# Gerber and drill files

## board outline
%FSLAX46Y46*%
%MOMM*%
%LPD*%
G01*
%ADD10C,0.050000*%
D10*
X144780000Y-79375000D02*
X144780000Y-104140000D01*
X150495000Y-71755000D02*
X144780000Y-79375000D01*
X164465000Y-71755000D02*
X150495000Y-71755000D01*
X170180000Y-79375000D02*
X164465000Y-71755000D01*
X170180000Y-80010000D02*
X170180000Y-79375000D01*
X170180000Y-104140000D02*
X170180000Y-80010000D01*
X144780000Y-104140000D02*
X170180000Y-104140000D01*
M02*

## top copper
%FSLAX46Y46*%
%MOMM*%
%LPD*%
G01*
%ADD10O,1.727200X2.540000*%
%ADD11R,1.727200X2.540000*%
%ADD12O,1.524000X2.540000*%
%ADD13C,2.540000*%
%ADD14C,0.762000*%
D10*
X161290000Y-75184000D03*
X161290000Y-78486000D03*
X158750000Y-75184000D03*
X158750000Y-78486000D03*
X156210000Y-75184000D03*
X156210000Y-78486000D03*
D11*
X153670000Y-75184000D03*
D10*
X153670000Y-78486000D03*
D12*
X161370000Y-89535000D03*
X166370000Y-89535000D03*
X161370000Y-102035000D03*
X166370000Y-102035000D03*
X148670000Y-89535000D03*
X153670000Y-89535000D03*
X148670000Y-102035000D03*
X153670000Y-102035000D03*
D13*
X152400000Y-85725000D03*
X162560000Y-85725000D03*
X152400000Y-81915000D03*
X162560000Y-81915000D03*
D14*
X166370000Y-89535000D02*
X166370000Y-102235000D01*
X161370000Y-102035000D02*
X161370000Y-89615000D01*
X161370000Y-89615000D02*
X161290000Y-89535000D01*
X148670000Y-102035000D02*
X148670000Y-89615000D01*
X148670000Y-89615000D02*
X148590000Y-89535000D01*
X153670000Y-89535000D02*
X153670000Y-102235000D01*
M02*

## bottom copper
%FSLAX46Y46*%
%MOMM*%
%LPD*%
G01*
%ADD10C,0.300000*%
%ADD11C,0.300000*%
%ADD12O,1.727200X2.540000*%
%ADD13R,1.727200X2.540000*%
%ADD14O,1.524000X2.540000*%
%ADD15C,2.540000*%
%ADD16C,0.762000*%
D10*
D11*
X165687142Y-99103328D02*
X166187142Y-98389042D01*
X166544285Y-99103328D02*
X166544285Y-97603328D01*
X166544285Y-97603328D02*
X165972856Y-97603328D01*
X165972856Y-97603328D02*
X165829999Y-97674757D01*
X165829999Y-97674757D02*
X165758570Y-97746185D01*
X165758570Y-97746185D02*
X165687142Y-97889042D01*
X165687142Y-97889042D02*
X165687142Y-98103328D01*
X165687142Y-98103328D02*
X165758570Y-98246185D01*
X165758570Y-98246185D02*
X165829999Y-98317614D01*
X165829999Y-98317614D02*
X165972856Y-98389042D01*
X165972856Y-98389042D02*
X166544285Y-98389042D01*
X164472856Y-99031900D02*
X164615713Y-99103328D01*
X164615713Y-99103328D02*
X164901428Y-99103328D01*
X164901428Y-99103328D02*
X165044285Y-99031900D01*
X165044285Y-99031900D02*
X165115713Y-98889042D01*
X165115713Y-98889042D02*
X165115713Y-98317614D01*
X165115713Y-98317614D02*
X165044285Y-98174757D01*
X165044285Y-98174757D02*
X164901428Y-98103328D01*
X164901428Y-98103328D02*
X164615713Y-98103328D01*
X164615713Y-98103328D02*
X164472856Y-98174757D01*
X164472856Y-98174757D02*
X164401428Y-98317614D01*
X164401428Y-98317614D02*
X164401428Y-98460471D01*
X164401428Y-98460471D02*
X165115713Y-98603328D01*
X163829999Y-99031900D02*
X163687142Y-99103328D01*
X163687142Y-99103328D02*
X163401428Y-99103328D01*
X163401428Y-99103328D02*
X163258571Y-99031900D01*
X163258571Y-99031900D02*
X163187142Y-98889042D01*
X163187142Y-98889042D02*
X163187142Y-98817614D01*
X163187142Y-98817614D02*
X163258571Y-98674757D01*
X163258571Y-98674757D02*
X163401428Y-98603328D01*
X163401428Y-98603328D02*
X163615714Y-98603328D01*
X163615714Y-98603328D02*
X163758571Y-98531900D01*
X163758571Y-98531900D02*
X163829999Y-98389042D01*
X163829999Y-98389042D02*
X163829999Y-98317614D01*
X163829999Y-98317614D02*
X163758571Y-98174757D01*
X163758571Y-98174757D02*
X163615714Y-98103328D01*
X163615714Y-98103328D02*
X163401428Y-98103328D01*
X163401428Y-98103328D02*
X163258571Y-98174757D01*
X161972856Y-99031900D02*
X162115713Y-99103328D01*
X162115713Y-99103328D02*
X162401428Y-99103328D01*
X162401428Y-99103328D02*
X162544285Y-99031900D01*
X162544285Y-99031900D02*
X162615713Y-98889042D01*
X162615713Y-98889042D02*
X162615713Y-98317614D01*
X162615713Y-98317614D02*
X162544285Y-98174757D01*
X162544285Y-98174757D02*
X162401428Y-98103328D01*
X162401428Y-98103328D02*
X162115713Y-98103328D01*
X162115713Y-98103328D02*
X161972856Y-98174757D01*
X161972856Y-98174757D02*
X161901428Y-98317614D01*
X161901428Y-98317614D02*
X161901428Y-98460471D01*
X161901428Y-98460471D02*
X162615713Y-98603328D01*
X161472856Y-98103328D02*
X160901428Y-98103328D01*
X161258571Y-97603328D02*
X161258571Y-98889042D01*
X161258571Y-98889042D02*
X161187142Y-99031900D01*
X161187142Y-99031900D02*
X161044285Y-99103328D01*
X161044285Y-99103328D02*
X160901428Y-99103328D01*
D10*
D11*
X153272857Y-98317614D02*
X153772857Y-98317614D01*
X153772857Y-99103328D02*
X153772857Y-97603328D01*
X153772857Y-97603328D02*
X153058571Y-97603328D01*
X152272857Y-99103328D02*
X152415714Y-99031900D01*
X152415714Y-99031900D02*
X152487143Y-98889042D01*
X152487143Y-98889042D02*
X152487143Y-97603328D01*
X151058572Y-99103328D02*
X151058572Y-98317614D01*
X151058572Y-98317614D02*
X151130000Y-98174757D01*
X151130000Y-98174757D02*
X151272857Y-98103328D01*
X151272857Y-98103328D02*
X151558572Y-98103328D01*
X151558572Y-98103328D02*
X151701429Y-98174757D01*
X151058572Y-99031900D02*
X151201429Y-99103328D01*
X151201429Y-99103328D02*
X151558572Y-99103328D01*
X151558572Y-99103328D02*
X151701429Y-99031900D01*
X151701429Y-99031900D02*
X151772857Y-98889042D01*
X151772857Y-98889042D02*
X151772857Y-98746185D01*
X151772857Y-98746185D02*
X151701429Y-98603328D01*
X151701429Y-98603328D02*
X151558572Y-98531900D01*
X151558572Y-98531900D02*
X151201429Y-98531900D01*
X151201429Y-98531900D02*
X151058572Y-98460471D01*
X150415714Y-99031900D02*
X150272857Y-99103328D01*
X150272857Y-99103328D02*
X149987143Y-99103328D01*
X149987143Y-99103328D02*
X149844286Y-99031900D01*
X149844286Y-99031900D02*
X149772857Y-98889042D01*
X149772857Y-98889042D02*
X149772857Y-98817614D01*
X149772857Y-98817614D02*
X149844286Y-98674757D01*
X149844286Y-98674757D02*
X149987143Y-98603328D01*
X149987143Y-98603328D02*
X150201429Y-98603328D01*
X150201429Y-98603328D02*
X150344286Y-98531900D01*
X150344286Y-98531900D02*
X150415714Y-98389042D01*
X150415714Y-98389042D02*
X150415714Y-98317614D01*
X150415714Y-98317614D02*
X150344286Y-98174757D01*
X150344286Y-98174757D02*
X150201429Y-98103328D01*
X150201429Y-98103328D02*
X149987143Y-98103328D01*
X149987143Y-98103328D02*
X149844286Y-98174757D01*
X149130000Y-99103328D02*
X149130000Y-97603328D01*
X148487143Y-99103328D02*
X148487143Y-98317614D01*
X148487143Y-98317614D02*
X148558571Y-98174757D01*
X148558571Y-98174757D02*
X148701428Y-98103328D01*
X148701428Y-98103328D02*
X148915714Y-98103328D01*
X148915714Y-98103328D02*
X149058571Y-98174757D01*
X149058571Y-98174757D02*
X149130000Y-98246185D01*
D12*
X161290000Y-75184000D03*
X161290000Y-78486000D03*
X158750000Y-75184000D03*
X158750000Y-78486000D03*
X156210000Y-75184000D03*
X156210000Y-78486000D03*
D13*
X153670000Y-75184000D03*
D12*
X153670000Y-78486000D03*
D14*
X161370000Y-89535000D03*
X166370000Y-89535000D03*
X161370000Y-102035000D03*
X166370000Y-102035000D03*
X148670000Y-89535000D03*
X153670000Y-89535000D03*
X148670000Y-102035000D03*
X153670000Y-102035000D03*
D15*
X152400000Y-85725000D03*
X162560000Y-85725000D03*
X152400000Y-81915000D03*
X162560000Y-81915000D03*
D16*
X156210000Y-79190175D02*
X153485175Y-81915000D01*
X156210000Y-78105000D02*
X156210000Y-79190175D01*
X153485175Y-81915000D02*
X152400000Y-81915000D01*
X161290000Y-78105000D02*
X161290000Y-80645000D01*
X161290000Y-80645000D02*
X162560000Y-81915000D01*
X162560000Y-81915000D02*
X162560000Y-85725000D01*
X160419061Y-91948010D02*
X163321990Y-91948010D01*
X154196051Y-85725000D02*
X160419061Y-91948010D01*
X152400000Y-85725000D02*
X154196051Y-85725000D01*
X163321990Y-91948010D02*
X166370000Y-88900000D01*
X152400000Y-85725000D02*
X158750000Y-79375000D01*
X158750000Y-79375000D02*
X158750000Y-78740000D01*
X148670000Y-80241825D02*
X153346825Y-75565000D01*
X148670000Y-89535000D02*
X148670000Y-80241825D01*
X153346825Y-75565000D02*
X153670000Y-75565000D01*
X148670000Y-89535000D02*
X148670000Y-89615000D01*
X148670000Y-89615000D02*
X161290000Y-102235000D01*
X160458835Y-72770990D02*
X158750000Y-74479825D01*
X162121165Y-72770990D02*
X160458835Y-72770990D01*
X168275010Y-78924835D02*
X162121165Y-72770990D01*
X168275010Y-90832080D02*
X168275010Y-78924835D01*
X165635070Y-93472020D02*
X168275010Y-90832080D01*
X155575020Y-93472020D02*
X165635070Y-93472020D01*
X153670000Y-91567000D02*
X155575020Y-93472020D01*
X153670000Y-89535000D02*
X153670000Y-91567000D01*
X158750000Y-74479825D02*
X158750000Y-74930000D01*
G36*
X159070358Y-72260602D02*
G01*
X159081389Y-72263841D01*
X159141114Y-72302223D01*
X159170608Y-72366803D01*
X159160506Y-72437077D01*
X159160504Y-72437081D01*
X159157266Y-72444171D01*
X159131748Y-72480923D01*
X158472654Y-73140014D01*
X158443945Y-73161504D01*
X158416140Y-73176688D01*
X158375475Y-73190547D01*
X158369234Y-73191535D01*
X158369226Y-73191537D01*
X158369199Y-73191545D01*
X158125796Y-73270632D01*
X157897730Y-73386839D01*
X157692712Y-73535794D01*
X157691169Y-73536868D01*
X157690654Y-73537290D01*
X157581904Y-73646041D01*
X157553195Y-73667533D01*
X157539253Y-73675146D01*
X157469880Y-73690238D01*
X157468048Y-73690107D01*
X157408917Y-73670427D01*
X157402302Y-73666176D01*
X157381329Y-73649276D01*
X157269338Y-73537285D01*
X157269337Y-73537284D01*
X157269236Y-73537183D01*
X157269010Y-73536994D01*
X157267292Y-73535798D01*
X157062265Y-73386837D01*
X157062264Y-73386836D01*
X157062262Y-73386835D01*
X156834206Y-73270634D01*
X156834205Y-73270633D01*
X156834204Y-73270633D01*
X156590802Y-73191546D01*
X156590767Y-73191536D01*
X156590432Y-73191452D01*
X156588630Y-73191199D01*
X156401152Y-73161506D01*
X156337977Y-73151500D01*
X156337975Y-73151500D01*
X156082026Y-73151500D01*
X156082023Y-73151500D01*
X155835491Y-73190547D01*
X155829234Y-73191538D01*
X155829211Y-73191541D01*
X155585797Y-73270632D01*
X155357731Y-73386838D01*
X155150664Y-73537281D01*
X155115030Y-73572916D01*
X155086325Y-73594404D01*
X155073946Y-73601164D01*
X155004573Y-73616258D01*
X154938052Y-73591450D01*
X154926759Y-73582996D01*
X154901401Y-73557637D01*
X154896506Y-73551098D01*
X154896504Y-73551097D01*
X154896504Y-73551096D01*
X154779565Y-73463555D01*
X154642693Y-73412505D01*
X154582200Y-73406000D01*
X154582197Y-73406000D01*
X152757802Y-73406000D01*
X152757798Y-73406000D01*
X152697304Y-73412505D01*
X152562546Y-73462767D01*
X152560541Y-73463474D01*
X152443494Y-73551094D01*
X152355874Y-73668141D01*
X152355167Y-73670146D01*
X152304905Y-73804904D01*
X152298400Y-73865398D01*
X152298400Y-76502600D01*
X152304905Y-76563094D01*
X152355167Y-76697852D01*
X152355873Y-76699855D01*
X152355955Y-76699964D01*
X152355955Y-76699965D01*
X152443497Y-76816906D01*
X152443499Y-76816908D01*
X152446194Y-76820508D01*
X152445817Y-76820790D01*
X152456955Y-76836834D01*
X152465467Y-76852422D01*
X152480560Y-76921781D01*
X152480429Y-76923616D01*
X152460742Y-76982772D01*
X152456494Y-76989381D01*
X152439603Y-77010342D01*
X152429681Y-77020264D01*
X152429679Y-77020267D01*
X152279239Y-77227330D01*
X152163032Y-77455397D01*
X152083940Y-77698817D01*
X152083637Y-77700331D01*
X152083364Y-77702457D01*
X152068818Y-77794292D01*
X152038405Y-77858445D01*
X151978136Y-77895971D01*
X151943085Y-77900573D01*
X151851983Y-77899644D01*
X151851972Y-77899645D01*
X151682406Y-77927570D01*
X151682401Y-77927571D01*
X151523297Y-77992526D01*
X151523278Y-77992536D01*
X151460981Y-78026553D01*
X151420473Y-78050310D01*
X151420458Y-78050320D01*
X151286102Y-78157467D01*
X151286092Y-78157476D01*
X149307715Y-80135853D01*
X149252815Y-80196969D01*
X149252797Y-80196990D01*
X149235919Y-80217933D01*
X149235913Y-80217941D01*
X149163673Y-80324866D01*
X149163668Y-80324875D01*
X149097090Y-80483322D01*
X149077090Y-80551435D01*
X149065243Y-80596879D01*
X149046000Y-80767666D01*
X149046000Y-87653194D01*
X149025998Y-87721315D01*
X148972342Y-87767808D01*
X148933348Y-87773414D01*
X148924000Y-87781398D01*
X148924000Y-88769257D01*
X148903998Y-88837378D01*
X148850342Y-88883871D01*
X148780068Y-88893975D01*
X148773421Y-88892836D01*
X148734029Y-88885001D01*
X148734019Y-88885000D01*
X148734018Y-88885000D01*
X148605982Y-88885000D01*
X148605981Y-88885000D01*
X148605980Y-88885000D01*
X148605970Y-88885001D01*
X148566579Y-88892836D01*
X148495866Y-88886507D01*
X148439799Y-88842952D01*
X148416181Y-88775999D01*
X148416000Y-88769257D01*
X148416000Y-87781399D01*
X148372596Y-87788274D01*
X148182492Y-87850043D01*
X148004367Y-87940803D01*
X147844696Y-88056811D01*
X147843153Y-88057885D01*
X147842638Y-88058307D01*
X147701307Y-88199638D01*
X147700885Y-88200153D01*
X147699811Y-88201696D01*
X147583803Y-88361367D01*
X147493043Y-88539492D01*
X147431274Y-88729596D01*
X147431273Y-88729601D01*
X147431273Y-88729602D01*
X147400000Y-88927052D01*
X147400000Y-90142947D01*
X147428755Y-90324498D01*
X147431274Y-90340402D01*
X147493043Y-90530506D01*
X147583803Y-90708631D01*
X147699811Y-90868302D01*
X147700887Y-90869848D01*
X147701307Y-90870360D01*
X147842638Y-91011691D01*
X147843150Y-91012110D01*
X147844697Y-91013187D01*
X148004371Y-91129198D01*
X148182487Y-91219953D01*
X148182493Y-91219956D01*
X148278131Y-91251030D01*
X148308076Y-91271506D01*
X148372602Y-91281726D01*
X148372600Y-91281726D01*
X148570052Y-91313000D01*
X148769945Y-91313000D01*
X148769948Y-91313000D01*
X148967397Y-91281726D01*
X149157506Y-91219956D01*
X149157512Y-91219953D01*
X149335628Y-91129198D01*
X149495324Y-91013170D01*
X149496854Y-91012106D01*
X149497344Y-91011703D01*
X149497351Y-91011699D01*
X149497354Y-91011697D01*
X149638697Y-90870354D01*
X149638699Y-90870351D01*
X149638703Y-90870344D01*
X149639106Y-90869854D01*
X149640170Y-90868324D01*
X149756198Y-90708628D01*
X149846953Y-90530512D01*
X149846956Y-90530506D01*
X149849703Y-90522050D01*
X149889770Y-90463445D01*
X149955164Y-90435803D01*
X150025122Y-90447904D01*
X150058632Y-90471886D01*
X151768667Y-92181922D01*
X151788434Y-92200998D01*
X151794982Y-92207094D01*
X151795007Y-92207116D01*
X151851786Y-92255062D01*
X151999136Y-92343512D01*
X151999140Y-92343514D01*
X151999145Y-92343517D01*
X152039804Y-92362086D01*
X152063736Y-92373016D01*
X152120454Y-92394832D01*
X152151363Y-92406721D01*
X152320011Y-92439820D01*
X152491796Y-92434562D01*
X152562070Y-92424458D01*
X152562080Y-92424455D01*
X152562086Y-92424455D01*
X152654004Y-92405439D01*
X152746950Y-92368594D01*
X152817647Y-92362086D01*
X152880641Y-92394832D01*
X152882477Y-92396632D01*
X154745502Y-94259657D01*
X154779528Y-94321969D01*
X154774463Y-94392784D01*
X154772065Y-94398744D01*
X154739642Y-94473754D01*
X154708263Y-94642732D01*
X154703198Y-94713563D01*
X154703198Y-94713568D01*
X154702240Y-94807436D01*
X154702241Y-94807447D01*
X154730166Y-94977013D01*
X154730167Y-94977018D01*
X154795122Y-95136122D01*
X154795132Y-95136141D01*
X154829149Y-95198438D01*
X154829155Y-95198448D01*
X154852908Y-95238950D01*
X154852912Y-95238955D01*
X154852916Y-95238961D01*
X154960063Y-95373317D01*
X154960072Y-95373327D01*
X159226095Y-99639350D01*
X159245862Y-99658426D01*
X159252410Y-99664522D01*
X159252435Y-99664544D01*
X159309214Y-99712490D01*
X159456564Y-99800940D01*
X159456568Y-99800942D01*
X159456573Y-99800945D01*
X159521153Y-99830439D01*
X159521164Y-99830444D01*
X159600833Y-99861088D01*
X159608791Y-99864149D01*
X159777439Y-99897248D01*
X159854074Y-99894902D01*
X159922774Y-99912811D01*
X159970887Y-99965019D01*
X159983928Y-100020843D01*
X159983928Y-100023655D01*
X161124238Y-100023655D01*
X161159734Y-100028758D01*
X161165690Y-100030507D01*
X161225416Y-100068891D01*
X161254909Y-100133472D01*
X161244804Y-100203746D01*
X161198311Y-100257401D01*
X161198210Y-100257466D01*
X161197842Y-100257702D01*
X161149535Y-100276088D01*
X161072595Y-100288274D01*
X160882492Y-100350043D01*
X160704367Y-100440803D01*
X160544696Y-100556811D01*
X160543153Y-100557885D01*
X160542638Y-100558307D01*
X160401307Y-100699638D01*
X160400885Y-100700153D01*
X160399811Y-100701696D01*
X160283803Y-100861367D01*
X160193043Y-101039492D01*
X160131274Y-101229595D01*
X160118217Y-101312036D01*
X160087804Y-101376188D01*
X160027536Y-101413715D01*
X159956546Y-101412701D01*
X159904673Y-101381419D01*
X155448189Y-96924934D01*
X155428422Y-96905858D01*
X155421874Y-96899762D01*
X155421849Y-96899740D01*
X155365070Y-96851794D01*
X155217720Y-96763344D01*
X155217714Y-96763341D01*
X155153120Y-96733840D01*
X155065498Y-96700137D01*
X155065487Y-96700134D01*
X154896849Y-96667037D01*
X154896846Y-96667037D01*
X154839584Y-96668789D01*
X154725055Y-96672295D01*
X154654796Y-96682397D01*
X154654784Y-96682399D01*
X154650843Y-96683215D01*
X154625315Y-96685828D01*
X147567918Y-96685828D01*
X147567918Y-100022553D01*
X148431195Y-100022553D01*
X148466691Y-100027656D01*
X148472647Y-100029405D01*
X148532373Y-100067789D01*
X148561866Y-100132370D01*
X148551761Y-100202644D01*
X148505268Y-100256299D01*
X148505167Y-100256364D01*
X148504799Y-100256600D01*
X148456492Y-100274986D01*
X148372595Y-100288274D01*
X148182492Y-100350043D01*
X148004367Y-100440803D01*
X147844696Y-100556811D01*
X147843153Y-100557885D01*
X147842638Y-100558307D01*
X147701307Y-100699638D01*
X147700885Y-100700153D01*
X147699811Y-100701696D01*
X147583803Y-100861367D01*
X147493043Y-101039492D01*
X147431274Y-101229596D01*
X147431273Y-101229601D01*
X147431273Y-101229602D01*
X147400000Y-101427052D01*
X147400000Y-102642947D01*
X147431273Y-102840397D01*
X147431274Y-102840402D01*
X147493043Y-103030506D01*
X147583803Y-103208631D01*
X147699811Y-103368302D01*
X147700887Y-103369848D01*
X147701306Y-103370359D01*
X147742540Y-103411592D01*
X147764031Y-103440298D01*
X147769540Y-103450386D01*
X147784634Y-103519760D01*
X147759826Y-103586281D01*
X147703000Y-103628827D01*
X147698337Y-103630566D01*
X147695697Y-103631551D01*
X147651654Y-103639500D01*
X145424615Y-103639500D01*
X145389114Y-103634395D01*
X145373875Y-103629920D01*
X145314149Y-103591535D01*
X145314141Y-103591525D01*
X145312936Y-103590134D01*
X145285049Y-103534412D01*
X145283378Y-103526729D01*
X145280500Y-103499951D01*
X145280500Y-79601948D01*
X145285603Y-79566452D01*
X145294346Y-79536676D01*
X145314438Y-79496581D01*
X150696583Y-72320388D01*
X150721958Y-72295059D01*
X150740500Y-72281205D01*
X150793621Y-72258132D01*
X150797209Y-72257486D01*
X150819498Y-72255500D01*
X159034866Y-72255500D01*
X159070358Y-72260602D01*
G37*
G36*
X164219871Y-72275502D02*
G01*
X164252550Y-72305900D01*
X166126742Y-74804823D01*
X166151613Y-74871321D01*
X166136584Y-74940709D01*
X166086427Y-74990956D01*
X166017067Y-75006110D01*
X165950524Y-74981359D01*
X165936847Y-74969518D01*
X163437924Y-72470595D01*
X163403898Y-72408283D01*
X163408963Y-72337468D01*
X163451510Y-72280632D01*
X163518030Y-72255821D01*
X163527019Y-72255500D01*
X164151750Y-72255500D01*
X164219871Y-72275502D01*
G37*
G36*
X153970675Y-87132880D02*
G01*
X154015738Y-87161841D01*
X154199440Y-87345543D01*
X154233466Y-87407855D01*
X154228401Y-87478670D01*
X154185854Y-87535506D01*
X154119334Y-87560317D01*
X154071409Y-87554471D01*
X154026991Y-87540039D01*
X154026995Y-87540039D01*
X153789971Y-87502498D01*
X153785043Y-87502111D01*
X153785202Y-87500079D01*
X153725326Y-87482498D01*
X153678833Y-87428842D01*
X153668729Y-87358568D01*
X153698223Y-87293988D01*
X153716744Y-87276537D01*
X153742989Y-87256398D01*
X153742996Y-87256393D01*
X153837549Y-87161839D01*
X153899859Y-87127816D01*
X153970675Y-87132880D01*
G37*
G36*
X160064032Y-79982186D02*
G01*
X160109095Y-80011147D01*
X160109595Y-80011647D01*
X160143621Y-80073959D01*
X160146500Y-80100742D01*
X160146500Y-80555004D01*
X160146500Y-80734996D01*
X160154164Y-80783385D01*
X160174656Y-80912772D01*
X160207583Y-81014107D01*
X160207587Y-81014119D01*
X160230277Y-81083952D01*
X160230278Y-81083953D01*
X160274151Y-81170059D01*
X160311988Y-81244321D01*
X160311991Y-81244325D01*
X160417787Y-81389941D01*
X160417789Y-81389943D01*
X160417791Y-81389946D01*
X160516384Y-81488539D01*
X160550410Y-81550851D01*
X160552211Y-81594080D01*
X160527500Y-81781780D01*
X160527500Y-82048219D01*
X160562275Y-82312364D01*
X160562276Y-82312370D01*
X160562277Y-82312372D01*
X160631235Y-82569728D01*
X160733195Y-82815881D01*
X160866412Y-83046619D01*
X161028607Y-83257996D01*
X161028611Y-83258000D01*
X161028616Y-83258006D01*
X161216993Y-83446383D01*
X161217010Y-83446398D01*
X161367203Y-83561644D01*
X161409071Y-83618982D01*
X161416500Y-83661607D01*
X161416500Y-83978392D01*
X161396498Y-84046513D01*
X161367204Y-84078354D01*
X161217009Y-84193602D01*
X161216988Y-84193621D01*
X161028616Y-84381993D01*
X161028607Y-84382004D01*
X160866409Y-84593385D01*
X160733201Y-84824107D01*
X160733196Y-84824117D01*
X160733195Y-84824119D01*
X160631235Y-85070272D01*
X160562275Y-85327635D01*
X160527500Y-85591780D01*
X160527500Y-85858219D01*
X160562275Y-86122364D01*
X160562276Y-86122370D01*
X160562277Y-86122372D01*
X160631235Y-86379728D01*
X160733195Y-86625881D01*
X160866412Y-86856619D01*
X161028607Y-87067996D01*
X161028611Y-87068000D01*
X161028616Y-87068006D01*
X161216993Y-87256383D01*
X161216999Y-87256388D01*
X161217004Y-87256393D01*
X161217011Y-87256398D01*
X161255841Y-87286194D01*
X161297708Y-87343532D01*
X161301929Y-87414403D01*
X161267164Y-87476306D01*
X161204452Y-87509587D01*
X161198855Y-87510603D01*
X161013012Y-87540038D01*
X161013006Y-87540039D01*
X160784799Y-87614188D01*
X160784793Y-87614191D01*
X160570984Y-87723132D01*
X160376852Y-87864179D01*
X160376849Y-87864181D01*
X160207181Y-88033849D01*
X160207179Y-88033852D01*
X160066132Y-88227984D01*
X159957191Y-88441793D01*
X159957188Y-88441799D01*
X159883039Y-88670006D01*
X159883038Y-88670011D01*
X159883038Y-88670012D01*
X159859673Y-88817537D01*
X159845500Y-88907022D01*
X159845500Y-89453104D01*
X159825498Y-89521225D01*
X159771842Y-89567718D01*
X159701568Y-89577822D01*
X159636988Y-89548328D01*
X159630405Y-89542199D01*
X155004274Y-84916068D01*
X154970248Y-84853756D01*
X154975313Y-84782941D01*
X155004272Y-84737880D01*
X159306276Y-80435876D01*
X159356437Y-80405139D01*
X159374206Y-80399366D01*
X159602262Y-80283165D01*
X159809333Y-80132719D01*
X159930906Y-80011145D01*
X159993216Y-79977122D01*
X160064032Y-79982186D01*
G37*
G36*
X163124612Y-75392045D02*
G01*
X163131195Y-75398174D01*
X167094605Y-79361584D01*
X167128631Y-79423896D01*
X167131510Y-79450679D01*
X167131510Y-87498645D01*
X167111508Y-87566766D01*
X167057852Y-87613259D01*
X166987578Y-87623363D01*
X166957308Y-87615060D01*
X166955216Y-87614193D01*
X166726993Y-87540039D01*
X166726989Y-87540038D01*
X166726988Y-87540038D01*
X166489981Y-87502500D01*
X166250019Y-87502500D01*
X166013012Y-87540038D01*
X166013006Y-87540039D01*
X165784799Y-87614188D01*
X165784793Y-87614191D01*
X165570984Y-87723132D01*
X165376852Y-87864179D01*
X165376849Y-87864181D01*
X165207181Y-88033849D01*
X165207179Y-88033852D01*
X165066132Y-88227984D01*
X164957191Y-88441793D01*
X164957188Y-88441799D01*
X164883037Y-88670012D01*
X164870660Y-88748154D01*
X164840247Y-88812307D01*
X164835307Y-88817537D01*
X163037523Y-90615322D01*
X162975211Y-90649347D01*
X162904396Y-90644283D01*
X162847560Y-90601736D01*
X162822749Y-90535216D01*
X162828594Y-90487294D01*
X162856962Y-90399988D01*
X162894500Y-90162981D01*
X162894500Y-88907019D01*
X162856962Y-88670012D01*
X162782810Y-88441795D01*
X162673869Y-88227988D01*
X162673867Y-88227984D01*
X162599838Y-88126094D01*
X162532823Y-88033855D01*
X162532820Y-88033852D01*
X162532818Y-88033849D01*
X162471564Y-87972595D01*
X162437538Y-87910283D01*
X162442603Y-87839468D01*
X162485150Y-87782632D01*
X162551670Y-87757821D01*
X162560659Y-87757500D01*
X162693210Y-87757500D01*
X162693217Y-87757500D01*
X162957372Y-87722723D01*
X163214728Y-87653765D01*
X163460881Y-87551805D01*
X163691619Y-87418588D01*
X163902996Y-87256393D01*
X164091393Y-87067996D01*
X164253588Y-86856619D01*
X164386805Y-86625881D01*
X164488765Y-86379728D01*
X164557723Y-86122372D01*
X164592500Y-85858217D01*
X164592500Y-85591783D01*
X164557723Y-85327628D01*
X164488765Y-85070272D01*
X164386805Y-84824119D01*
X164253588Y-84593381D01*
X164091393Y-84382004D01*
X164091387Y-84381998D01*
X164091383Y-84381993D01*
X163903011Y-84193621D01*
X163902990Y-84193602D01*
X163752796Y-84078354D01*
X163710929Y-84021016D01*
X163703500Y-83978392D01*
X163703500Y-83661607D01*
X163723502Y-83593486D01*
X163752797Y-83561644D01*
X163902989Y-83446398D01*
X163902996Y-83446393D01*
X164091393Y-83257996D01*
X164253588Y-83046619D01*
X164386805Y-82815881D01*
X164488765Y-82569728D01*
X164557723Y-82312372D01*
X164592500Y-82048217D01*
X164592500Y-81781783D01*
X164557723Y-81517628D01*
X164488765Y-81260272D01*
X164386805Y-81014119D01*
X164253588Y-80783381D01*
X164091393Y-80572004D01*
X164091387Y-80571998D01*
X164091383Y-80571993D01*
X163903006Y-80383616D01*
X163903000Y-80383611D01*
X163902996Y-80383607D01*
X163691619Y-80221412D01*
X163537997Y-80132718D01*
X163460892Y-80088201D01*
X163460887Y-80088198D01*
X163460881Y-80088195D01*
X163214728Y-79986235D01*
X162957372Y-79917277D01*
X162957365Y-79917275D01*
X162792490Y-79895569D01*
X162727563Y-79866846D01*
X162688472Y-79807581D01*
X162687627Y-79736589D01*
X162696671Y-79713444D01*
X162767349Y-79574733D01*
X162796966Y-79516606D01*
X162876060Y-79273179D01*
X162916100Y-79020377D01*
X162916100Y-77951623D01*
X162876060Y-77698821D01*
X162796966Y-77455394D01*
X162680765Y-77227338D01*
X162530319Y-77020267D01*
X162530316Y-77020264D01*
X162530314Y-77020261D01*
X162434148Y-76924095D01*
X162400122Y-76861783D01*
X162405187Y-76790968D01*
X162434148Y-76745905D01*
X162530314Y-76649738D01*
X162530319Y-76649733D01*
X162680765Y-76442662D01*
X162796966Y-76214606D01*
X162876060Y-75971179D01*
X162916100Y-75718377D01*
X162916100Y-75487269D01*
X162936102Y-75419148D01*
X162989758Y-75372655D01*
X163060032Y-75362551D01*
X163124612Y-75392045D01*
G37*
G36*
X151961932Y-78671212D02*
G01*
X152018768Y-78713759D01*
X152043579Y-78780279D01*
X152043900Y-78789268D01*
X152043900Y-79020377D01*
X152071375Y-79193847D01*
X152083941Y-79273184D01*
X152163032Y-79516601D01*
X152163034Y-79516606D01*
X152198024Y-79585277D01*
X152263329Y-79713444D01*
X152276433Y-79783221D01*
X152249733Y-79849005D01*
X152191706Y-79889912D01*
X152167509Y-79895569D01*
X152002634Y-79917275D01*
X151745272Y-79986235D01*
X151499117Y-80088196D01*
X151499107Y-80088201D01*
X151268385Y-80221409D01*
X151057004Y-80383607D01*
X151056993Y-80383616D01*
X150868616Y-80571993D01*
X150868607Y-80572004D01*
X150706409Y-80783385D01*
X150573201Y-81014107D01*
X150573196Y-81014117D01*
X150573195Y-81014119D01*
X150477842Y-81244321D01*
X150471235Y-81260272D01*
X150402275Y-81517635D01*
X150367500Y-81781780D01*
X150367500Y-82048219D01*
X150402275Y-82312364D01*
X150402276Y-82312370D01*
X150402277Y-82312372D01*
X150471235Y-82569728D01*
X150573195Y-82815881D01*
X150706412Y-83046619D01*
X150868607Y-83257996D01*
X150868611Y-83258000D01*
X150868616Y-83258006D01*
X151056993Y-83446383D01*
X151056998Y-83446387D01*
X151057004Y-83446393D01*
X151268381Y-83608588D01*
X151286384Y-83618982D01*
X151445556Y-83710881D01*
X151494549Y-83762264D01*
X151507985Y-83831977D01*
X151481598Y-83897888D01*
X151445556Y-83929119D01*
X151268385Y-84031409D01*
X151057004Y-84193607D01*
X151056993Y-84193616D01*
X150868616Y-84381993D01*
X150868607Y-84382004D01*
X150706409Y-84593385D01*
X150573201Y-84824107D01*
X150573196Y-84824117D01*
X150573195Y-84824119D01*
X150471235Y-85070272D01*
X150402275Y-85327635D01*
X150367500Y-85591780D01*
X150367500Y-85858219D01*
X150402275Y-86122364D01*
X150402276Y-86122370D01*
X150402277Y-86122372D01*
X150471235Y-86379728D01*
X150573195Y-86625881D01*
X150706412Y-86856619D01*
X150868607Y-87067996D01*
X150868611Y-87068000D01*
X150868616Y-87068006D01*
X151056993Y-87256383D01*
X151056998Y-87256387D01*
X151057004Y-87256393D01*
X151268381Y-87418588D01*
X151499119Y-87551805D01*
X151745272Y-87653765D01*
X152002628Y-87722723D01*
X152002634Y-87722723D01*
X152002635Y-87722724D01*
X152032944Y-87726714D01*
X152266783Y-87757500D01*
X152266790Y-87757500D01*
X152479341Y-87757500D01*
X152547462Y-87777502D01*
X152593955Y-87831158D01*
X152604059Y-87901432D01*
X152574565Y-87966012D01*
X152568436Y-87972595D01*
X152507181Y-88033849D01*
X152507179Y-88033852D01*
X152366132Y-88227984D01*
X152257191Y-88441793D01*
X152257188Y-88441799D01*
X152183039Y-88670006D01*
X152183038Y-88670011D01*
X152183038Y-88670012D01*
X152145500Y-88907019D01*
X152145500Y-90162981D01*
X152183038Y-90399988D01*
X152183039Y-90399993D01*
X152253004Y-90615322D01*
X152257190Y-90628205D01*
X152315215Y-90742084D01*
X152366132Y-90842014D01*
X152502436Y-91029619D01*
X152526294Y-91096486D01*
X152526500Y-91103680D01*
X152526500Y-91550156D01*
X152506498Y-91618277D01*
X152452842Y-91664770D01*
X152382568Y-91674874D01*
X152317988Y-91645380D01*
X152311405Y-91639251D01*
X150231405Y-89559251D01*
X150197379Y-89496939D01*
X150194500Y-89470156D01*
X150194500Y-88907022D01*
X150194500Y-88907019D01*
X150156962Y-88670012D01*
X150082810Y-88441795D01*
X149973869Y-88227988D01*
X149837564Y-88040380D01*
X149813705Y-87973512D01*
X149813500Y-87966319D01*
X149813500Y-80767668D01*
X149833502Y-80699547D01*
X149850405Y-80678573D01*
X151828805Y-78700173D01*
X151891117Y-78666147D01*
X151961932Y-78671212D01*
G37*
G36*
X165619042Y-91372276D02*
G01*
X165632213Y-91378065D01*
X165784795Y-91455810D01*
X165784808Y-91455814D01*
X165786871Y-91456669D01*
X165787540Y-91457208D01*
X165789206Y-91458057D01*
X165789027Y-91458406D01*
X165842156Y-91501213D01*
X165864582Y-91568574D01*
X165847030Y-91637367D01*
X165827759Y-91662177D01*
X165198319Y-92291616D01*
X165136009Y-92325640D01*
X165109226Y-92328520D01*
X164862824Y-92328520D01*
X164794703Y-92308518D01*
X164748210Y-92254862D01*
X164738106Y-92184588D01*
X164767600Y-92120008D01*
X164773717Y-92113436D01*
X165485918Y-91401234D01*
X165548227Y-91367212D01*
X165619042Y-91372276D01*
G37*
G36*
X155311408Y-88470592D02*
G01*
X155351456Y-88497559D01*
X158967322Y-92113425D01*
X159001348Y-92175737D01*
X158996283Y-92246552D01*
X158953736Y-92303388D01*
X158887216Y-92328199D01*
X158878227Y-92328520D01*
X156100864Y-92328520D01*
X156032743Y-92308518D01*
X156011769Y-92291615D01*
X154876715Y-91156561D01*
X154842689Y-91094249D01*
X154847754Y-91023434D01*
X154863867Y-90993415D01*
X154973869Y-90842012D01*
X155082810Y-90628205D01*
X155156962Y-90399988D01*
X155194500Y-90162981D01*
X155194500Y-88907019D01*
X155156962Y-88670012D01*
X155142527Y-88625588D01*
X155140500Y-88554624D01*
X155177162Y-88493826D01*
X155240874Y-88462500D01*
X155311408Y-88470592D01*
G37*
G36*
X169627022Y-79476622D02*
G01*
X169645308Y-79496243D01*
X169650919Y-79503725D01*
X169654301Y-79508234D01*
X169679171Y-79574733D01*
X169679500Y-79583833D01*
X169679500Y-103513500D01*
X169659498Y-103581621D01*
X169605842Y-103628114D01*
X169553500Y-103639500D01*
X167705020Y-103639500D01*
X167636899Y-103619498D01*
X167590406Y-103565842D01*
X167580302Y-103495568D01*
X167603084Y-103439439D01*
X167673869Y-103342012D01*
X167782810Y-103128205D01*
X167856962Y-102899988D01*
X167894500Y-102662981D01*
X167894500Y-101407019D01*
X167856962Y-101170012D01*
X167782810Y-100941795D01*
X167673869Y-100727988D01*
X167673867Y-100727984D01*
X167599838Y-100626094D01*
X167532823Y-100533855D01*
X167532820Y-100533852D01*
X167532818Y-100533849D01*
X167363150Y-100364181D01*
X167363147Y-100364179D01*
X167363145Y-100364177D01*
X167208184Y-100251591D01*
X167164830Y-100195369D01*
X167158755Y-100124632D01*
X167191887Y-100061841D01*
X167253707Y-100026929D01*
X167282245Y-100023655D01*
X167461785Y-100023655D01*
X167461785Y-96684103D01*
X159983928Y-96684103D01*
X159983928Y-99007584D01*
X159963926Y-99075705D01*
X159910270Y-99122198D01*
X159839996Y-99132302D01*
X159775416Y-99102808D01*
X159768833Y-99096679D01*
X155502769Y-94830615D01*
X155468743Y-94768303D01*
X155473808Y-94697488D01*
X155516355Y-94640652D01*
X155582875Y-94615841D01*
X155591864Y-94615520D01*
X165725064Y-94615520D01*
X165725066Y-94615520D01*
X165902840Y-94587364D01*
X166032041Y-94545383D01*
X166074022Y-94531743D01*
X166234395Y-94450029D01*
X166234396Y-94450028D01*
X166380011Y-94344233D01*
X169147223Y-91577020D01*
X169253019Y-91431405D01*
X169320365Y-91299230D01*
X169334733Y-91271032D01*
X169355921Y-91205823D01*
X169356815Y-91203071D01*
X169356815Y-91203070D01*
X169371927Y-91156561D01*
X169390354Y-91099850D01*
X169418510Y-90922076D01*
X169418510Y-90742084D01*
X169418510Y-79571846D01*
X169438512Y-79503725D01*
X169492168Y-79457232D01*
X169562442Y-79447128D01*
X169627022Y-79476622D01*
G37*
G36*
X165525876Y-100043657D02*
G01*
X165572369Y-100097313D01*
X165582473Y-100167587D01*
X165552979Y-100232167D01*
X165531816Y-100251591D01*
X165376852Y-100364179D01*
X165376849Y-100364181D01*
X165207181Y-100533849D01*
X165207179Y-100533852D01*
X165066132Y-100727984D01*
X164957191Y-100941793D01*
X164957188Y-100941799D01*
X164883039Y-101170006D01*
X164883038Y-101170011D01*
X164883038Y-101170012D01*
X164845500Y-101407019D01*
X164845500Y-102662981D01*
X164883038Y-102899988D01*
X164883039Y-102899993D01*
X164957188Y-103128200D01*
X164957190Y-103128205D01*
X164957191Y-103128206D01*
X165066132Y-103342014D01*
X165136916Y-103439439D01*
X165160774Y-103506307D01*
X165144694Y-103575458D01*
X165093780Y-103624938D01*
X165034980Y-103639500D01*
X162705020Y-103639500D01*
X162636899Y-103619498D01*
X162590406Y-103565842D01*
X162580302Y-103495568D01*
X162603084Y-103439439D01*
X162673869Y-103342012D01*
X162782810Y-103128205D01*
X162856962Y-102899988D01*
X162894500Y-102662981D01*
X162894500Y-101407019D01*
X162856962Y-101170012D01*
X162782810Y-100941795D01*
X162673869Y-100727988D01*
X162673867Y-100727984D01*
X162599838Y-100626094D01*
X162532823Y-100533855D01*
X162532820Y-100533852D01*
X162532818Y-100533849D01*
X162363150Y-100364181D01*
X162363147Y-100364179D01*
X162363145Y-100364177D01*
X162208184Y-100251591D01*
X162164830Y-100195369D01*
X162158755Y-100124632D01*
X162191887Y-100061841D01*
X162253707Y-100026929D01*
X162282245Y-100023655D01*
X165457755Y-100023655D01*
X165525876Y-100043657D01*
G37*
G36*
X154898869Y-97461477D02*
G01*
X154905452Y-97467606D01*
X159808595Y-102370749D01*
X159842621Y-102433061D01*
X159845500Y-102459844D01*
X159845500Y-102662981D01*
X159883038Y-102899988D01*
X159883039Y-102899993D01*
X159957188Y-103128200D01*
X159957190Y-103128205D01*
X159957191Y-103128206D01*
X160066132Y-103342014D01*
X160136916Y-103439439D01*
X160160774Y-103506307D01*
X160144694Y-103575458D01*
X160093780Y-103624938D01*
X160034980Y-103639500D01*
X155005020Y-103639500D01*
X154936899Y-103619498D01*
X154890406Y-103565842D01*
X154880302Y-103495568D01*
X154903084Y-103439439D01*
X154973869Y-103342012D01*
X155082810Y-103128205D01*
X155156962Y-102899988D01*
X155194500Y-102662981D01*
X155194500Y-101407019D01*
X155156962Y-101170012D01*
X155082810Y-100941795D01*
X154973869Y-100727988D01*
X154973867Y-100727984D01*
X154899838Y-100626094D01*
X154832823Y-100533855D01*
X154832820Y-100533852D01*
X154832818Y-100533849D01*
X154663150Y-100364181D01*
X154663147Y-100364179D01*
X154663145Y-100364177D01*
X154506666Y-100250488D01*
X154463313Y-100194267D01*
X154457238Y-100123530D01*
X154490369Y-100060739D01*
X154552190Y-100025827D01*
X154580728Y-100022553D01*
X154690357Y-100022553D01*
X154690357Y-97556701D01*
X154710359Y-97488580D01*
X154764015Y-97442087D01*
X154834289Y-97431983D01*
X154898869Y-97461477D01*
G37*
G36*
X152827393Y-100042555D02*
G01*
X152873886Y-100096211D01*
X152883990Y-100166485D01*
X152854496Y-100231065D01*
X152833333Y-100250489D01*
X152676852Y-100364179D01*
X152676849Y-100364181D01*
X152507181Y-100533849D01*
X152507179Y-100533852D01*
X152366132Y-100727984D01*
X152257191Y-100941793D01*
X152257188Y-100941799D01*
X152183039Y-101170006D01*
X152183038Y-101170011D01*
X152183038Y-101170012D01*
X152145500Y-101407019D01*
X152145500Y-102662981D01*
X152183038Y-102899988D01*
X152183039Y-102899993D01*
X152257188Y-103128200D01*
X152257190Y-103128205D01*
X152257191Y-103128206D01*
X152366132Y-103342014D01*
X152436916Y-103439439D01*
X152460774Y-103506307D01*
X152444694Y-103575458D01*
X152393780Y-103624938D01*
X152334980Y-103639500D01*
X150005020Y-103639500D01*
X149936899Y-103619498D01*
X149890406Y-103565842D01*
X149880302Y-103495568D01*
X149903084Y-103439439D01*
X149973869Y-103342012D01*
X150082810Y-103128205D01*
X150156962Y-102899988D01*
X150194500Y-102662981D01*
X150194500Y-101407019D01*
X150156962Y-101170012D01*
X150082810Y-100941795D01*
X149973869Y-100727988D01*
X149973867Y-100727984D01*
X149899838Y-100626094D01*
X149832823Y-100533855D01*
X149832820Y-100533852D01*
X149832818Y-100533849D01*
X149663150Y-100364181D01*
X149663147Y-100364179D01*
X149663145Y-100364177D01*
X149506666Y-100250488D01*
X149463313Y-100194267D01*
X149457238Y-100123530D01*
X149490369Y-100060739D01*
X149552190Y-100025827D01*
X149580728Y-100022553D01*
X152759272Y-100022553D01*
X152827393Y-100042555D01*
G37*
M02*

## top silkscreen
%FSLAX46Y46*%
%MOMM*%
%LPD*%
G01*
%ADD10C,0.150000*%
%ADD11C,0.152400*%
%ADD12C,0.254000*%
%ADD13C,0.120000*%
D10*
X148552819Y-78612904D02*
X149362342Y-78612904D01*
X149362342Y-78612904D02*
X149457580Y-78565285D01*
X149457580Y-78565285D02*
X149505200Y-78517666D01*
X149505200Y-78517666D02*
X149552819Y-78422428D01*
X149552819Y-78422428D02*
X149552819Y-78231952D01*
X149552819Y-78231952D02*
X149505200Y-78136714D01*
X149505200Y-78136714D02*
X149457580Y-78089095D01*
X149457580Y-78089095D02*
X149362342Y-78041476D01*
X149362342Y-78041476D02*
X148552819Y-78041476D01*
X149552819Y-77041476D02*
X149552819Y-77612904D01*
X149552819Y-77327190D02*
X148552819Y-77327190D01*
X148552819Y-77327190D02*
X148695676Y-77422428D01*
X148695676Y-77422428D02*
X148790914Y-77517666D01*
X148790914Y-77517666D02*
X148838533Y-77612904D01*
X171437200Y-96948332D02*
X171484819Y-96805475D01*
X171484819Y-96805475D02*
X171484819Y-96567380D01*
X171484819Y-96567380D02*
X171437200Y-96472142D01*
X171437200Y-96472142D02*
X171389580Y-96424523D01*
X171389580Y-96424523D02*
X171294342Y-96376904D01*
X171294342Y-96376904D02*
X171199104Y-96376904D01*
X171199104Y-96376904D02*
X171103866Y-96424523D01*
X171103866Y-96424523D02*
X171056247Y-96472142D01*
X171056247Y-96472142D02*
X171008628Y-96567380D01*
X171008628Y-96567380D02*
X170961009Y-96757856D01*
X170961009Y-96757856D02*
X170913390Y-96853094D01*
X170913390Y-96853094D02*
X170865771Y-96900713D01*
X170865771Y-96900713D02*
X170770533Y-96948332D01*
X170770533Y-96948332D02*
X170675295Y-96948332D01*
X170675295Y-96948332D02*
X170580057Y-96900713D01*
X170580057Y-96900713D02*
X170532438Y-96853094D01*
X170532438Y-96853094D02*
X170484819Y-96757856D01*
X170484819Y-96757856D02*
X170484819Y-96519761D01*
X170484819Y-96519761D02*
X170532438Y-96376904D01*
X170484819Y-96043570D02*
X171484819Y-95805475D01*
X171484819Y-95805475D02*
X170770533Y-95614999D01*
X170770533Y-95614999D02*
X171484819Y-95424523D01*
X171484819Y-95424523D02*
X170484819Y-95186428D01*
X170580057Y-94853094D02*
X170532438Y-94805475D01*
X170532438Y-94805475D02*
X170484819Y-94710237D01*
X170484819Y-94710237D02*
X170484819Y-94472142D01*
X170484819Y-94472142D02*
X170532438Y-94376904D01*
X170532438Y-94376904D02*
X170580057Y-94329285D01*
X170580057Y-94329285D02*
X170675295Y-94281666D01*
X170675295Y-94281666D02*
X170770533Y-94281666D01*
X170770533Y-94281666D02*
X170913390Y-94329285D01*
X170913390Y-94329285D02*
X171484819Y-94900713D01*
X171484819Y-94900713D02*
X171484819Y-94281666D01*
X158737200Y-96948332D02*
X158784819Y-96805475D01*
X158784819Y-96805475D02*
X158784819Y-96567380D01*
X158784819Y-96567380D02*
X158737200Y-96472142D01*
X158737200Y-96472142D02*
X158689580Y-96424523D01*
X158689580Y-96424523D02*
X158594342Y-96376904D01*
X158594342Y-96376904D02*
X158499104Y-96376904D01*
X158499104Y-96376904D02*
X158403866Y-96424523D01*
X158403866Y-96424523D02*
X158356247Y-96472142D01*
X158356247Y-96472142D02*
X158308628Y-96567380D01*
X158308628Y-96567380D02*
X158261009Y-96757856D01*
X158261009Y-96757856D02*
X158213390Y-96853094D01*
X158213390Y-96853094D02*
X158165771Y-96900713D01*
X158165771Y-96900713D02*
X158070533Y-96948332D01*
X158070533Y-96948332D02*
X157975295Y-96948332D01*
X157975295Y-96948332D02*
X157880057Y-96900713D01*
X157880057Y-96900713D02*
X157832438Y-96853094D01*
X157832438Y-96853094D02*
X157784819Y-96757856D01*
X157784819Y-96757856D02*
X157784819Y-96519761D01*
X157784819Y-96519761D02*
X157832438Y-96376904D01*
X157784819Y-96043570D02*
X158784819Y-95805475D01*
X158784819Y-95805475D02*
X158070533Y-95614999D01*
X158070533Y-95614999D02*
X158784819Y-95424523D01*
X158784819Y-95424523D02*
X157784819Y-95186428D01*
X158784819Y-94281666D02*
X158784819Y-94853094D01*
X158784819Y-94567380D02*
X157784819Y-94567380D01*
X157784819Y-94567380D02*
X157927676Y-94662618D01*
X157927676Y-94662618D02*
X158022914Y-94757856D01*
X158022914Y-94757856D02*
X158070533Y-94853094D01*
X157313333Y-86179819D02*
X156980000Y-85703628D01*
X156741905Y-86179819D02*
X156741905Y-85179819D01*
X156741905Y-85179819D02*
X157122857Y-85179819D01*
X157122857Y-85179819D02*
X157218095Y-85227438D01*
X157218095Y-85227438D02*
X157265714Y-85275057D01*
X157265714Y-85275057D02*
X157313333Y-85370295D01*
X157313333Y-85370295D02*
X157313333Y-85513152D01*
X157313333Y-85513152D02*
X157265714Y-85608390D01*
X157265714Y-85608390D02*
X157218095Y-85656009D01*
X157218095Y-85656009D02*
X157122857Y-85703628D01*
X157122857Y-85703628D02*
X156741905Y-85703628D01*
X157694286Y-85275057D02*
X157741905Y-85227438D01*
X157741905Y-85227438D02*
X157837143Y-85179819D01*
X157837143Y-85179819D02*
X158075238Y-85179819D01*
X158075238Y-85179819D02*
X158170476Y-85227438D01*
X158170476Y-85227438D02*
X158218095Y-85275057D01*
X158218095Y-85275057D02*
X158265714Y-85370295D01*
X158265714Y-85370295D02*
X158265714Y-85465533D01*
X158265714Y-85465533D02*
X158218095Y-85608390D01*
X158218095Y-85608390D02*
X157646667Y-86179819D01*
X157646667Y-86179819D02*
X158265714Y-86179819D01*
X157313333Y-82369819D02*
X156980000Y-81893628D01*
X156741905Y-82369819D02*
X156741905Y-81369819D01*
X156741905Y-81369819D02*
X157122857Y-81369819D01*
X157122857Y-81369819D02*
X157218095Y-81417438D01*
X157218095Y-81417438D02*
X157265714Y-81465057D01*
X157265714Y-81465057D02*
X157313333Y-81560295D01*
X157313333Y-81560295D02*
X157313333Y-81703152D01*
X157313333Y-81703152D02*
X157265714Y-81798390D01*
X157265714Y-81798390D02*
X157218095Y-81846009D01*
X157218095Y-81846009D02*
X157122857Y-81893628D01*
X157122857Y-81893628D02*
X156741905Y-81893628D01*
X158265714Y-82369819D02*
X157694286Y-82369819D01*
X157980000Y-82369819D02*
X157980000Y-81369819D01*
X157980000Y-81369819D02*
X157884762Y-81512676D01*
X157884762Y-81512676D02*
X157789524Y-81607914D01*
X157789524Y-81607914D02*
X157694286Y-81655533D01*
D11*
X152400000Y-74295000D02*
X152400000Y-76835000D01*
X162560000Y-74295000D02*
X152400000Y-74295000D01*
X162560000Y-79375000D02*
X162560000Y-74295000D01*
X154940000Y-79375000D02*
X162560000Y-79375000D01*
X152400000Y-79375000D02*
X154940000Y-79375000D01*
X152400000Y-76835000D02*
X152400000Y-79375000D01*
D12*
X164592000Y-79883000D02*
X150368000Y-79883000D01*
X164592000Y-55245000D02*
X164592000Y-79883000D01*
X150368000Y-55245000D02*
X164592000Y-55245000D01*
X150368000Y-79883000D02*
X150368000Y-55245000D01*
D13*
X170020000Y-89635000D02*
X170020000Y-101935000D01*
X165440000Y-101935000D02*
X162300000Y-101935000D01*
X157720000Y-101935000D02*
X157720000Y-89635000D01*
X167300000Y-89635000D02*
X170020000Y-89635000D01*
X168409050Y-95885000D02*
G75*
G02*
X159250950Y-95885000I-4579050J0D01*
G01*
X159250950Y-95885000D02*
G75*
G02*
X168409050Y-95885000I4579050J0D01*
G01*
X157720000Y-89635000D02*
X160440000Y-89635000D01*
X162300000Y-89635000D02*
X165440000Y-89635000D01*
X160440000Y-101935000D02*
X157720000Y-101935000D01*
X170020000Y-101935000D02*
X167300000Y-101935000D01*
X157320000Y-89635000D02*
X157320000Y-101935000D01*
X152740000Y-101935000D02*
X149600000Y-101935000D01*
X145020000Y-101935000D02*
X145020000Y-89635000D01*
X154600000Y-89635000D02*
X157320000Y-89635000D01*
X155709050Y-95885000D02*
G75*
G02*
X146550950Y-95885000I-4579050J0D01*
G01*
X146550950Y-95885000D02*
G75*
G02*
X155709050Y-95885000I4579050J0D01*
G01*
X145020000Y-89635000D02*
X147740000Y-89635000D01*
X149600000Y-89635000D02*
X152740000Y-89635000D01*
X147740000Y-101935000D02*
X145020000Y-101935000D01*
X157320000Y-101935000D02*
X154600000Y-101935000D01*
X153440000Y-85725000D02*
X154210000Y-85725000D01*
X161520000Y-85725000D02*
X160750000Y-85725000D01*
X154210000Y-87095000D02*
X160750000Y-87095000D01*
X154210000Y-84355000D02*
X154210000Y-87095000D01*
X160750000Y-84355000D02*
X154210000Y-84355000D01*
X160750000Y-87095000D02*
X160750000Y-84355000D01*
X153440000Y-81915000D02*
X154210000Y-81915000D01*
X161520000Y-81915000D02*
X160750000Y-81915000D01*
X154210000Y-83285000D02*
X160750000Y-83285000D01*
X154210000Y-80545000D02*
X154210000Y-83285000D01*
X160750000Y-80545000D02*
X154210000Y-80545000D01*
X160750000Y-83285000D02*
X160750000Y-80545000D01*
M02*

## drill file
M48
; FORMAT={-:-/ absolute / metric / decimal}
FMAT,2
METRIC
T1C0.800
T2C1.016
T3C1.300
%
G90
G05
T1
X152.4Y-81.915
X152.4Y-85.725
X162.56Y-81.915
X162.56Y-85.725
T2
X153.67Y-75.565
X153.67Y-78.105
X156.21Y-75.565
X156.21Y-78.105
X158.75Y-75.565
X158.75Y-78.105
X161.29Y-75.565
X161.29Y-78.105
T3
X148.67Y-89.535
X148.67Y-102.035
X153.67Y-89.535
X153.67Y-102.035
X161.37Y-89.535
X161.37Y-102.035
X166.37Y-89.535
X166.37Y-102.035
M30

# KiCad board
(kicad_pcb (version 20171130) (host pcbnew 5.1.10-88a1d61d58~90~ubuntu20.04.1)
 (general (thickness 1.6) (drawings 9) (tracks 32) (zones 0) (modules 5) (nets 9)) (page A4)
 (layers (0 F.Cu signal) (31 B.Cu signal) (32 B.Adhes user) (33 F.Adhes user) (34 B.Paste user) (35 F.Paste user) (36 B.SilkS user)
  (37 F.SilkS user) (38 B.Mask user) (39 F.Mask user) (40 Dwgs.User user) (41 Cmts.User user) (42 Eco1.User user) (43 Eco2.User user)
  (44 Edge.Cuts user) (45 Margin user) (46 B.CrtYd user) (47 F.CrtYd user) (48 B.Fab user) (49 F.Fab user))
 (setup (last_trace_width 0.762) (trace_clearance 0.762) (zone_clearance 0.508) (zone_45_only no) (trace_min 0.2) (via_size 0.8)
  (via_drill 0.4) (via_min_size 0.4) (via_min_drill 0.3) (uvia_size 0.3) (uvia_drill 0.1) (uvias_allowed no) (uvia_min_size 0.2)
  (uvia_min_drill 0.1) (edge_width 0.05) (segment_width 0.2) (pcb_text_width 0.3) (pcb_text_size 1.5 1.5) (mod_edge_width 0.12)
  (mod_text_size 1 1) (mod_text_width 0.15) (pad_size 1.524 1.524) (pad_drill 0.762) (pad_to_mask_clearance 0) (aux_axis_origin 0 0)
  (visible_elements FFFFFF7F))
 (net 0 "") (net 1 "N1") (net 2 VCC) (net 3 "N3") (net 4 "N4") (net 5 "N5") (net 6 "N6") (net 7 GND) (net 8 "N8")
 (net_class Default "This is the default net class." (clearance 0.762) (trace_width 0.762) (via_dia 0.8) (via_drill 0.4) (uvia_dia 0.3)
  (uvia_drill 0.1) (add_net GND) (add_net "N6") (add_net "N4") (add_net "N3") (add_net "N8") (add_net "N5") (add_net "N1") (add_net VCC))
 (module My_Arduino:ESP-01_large (layer F.Cu) (at 153.67 78.105 90)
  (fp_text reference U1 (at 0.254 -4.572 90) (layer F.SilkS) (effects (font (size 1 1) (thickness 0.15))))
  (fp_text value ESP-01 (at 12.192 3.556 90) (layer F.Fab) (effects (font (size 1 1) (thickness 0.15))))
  (fp_line (start 3.81 -1.27) (end 1.27 -1.27) (layer F.SilkS) (width 0.1524))
  (fp_line (start 3.81 8.89) (end 3.81 -1.27) (layer F.SilkS) (width 0.1524))
  (fp_line (start -1.27 8.89) (end 3.81 8.89) (layer F.SilkS) (width 0.1524))
  (fp_line (start -1.27 1.27) (end -1.27 8.89) (layer F.SilkS) (width 0.1524))
  (fp_line (start -1.27 -1.27) (end -1.27 1.27) (layer F.SilkS) (width 0.1524))
  (fp_line (start 1.27 -1.27) (end -1.27 -1.27) (layer F.SilkS) (width 0.1524))
  (fp_line (start -1.778 10.922) (end -1.778 -3.302) (layer F.SilkS) (width 0.254))
  (fp_line (start 22.86 10.922) (end -1.778 10.922) (layer F.SilkS) (width 0.254))
  (fp_line (start 22.86 -3.302) (end 22.86 10.922) (layer F.SilkS) (width 0.254))
  (fp_line (start -1.778 -3.302) (end 22.86 -3.302) (layer F.SilkS) (width 0.254))
  (pad 7 thru_hole oval (at 2.54 7.62 90) (size 2.54 1.7272) (drill 1.016 (offset 0.381 0)) (layers *.Cu *.Mask) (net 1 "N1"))
  (pad 8 thru_hole oval (at 0 7.62 90) (size 2.54 1.7272) (drill 1.016 (offset -0.381 0)) (layers *.Cu *.Mask) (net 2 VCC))
  (pad 5 thru_hole oval (at 2.54 5.08 90) (size 2.54 1.7272) (drill 1.016 (offset 0.381 0)) (layers *.Cu *.Mask) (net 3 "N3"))
  (pad 6 thru_hole oval (at 0 5.08 90) (size 2.54 1.7272) (drill 1.016 (offset -0.381 0)) (layers *.Cu *.Mask) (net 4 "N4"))
  (pad 3 thru_hole oval (at 2.54 2.54 90) (size 2.54 1.7272) (drill 1.016 (offset 0.381 0)) (layers *.Cu *.Mask) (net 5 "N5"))
  (pad 4 thru_hole oval (at 0 2.54 90) (size 2.54 1.7272) (drill 1.016 (offset -0.381 0)) (layers *.Cu *.Mask) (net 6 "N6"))
  (pad 1 thru_hole rect (at 2.54 0 90) (size 2.54 1.7272) (drill 1.016 (offset 0.381 0)) (layers *.Cu *.Mask) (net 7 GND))
  (pad 2 thru_hole oval (at 0 0 90) (size 2.54 1.7272) (drill 1.016 (offset -0.381 0)) (layers *.Cu *.Mask) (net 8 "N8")))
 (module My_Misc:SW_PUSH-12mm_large (layer F.Cu) (at 166.37 89.535 270)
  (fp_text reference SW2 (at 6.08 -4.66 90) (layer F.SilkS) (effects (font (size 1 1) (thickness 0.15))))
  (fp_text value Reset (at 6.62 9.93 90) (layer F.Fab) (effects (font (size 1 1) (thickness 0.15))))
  (fp_line (start 0.1 -3.65) (end 12.4 -3.65) (layer F.SilkS) (width 0.12))
  (fp_line (start 12.4 0.93) (end 12.4 4.07) (layer F.SilkS) (width 0.12))
  (fp_line (start 12.4 8.65) (end 0.1 8.65) (layer F.SilkS) (width 0.12))
  (fp_line (start 0.1 -0.93) (end 0.1 -3.65) (layer F.SilkS) (width 0.12))
  (fp_circle (center 6.35 2.54) (end 10.16 5.08) (layer F.SilkS) (width 0.12))
  (fp_line (start 0.1 8.65) (end 0.1 5.93) (layer F.SilkS) (width 0.12))
  (fp_line (start 0.1 4.07) (end 0.1 0.93) (layer F.SilkS) (width 0.12))
  (fp_line (start 12.4 5.93) (end 12.4 8.65) (layer F.SilkS) (width 0.12))
  (fp_line (start 12.4 -3.65) (end 12.4 -0.93) (layer F.SilkS) (width 0.12))
  (pad 2 thru_hole oval (at 0 5 270) (size 2.54 1.524) (drill 1.3) (layers *.Cu *.Mask) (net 7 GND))
  (pad 1 thru_hole oval (at 0 0 270) (size 2.54 1.524) (drill 1.3) (layers *.Cu *.Mask) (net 4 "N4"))
  (pad 2 thru_hole oval (at 12.5 5 270) (size 2.54 1.524) (drill 1.3) (layers *.Cu *.Mask) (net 7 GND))
  (pad 1 thru_hole oval (at 12.5 0 270) (size 2.54 1.524) (drill 1.3) (layers *.Cu *.Mask) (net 4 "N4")))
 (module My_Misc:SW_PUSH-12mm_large (layer F.Cu) (at 153.67 89.535 270)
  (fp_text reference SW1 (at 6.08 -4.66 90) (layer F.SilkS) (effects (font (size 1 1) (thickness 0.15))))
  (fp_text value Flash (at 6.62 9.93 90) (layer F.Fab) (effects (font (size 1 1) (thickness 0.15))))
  (fp_line (start 0.1 -3.65) (end 12.4 -3.65) (layer F.SilkS) (width 0.12))
  (fp_line (start 12.4 0.93) (end 12.4 4.07) (layer F.SilkS) (width 0.12))
  (fp_line (start 12.4 8.65) (end 0.1 8.65) (layer F.SilkS) (width 0.12))
  (fp_line (start 0.1 -0.93) (end 0.1 -3.65) (layer F.SilkS) (width 0.12))
  (fp_circle (center 6.35 2.54) (end 10.16 5.08) (layer F.SilkS) (width 0.12))
  (fp_line (start 0.1 8.65) (end 0.1 5.93) (layer F.SilkS) (width 0.12))
  (fp_line (start 0.1 4.07) (end 0.1 0.93) (layer F.SilkS) (width 0.12))
  (fp_line (start 12.4 5.93) (end 12.4 8.65) (layer F.SilkS) (width 0.12))
  (fp_line (start 12.4 -3.65) (end 12.4 -0.93) (layer F.SilkS) (width 0.12))
  (pad 2 thru_hole oval (at 0 5 270) (size 2.54 1.524) (drill 1.3) (layers *.Cu *.Mask) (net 7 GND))
  (pad 1 thru_hole oval (at 0 0 270) (size 2.54 1.524) (drill 1.3) (layers *.Cu *.Mask) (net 3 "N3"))
  (pad 2 thru_hole oval (at 12.5 5 270) (size 2.54 1.524) (drill 1.3) (layers *.Cu *.Mask) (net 7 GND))
  (pad 1 thru_hole oval (at 12.5 0 270) (size 2.54 1.524) (drill 1.3) (layers *.Cu *.Mask) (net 3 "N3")))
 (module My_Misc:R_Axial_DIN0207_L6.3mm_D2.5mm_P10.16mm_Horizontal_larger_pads (layer F.Cu) (at 162.56 85.725 180)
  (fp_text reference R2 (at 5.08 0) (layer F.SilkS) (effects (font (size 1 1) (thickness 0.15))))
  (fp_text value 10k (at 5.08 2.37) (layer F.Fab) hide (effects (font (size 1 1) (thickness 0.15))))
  (fp_line (start 9.12 0) (end 8.35 0) (layer F.SilkS) (width 0.12))
  (fp_line (start 1.04 0) (end 1.81 0) (layer F.SilkS) (width 0.12))
  (fp_line (start 8.35 -1.37) (end 1.81 -1.37) (layer F.SilkS) (width 0.12))
  (fp_line (start 8.35 1.37) (end 8.35 -1.37) (layer F.SilkS) (width 0.12))
  (fp_line (start 1.81 1.37) (end 8.35 1.37) (layer F.SilkS) (width 0.12))
  (fp_line (start 1.81 -1.37) (end 1.81 1.37) (layer F.SilkS) (width 0.12))
  (pad 2 thru_hole circle (at 10.16 0 180) (size 2.54 2.54) (drill 0.8) (layers *.Cu *.Mask) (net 4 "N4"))
  (pad 1 thru_hole circle (at 0 0 180) (size 2.54 2.54) (drill 0.8) (layers *.Cu *.Mask) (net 2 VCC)))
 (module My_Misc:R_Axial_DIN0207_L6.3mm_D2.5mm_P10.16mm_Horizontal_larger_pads (layer F.Cu) (at 162.56 81.915 180)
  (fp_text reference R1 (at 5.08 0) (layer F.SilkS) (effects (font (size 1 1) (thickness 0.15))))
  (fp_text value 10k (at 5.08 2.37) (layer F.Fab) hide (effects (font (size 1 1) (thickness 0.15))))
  (fp_line (start 9.12 0) (end 8.35 0) (layer F.SilkS) (width 0.12))
  (fp_line (start 1.04 0) (end 1.81 0) (layer F.SilkS) (width 0.12))
  (fp_line (start 8.35 -1.37) (end 1.81 -1.37) (layer F.SilkS) (width 0.12))
  (fp_line (start 8.35 1.37) (end 8.35 -1.37) (layer F.SilkS) (width 0.12))
  (fp_line (start 1.81 1.37) (end 8.35 1.37) (layer F.SilkS) (width 0.12))
  (fp_line (start 1.81 -1.37) (end 1.81 1.37) (layer F.SilkS) (width 0.12))
  (pad 2 thru_hole circle (at 10.16 0 180) (size 2.54 2.54) (drill 0.8) (layers *.Cu *.Mask) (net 6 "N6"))
  (pad 1 thru_hole circle (at 0 0 180) (size 2.54 2.54) (drill 0.8) (layers *.Cu *.Mask) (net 2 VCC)))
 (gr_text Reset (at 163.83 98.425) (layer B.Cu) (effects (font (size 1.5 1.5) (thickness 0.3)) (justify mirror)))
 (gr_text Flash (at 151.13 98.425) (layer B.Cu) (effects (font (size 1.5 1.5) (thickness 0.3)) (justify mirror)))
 (gr_line (start 144.78 79.375) (end 144.78 104.14) (layer Edge.Cuts) (width 0.05))
 (gr_line (start 150.495 71.755) (end 144.78 79.375) (layer Edge.Cuts) (width 0.05))
 (gr_line (start 164.465 71.755) (end 150.495 71.755) (layer Edge.Cuts) (width 0.05))
 (gr_line (start 170.18 79.375) (end 164.465 71.755) (layer Edge.Cuts) (width 0.05))
 (gr_line (start 170.18 80.01) (end 170.18 79.375) (layer Edge.Cuts) (width 0.05))
 (gr_line (start 170.18 104.14) (end 170.18 80.01) (layer Edge.Cuts) (width 0.05))
 (gr_line (start 144.78 104.14) (end 170.18 104.14) (layer Edge.Cuts) (width 0.05))
 (segment (start 156.21 79.190175) (end 153.485175 81.915) (width 0.762) (layer B.Cu) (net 6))
 (segment (start 156.21 78.105) (end 156.21 79.190175) (width 0.762) (layer B.Cu) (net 6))
 (segment (start 153.485175 81.915) (end 152.4 81.915) (width 0.762) (layer B.Cu) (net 6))
 (segment (start 161.29 78.105) (end 161.29 80.645) (width 0.762) (layer B.Cu) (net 2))
 (segment (start 161.29 80.645) (end 162.56 81.915) (width 0.762) (layer B.Cu) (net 2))
 (segment (start 162.56 81.915) (end 162.56 85.725) (width 0.762) (layer B.Cu) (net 2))
 (segment (start 166.37 89.535) (end 166.37 102.235) (width 0.762) (layer F.Cu) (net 4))
 (segment (start 160.419061 91.94801) (end 163.32199 91.94801) (width 0.762) (layer B.Cu) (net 4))
 (segment (start 154.196051 85.725) (end 160.419061 91.94801) (width 0.762) (layer B.Cu) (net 4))
 (segment (start 152.4 85.725) (end 154.196051 85.725) (width 0.762) (layer B.Cu) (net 4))
 (segment (start 163.32199 91.94801) (end 166.37 88.9) (width 0.762) (layer B.Cu) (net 4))
 (segment (start 152.4 85.725) (end 158.75 79.375) (width 0.762) (layer B.Cu) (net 4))
 (segment (start 158.75 79.375) (end 158.75 78.74) (width 0.762) (layer B.Cu) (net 4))
 (segment (start 161.37 102.035) (end 161.37 89.615) (width 0.762) (layer F.Cu) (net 7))
 (segment (start 161.37 89.615) (end 161.29 89.535) (width 0.762) (layer F.Cu) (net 7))
 (segment (start 148.67 102.035) (end 148.67 89.615) (width 0.762) (layer F.Cu) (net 7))
 (segment (start 148.67 89.615) (end 148.59 89.535) (width 0.762) (layer F.Cu) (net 7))
 (segment (start 148.67 80.241825) (end 153.346825 75.565) (width 0.762) (layer B.Cu) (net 7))
 (segment (start 148.67 89.535) (end 148.67 80.241825) (width 0.762) (layer B.Cu) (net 7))
 (segment (start 153.346825 75.565) (end 153.67 75.565) (width 0.762) (layer B.Cu) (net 7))
 (segment (start 148.67 89.535) (end 148.67 89.615) (width 0.762) (layer B.Cu) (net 7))
 (segment (start 148.67 89.615) (end 161.29 102.235) (width 0.762) (layer B.Cu) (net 7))
 (segment (start 153.67 89.535) (end 153.67 102.235) (width 0.762) (layer F.Cu) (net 3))
 (segment (start 160.458835 72.77099) (end 158.75 74.479825) (width 0.762) (layer B.Cu) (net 3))
 (segment (start 162.121165 72.77099) (end 160.458835 72.77099) (width 0.762) (layer B.Cu) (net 3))
 (segment (start 168.27501 78.924835) (end 162.121165 72.77099) (width 0.762) (layer B.Cu) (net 3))
 (segment (start 168.27501 90.83208) (end 168.27501 78.924835) (width 0.762) (layer B.Cu) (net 3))
 (segment (start 165.63507 93.47202) (end 168.27501 90.83208) (width 0.762) (layer B.Cu) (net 3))
 (segment (start 155.57502 93.47202) (end 165.63507 93.47202) (width 0.762) (layer B.Cu) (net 3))
 (segment (start 153.67 91.567) (end 155.57502 93.47202) (width 0.762) (layer B.Cu) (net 3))
 (segment (start 153.67 89.535) (end 153.67 91.567) (width 0.762) (layer B.Cu) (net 3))
 (segment (start 158.75 74.479825) (end 158.75 74.93) (width 0.762) (layer B.Cu) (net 3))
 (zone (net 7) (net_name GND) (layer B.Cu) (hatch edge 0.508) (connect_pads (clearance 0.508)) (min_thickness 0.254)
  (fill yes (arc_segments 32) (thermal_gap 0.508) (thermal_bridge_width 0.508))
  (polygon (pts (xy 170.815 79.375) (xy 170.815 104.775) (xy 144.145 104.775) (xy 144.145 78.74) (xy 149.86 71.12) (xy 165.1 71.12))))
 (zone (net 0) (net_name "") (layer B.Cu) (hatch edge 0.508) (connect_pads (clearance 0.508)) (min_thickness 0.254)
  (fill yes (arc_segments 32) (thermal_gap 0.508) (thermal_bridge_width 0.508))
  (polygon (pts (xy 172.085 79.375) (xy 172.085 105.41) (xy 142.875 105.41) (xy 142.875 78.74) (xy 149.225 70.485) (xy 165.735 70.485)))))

